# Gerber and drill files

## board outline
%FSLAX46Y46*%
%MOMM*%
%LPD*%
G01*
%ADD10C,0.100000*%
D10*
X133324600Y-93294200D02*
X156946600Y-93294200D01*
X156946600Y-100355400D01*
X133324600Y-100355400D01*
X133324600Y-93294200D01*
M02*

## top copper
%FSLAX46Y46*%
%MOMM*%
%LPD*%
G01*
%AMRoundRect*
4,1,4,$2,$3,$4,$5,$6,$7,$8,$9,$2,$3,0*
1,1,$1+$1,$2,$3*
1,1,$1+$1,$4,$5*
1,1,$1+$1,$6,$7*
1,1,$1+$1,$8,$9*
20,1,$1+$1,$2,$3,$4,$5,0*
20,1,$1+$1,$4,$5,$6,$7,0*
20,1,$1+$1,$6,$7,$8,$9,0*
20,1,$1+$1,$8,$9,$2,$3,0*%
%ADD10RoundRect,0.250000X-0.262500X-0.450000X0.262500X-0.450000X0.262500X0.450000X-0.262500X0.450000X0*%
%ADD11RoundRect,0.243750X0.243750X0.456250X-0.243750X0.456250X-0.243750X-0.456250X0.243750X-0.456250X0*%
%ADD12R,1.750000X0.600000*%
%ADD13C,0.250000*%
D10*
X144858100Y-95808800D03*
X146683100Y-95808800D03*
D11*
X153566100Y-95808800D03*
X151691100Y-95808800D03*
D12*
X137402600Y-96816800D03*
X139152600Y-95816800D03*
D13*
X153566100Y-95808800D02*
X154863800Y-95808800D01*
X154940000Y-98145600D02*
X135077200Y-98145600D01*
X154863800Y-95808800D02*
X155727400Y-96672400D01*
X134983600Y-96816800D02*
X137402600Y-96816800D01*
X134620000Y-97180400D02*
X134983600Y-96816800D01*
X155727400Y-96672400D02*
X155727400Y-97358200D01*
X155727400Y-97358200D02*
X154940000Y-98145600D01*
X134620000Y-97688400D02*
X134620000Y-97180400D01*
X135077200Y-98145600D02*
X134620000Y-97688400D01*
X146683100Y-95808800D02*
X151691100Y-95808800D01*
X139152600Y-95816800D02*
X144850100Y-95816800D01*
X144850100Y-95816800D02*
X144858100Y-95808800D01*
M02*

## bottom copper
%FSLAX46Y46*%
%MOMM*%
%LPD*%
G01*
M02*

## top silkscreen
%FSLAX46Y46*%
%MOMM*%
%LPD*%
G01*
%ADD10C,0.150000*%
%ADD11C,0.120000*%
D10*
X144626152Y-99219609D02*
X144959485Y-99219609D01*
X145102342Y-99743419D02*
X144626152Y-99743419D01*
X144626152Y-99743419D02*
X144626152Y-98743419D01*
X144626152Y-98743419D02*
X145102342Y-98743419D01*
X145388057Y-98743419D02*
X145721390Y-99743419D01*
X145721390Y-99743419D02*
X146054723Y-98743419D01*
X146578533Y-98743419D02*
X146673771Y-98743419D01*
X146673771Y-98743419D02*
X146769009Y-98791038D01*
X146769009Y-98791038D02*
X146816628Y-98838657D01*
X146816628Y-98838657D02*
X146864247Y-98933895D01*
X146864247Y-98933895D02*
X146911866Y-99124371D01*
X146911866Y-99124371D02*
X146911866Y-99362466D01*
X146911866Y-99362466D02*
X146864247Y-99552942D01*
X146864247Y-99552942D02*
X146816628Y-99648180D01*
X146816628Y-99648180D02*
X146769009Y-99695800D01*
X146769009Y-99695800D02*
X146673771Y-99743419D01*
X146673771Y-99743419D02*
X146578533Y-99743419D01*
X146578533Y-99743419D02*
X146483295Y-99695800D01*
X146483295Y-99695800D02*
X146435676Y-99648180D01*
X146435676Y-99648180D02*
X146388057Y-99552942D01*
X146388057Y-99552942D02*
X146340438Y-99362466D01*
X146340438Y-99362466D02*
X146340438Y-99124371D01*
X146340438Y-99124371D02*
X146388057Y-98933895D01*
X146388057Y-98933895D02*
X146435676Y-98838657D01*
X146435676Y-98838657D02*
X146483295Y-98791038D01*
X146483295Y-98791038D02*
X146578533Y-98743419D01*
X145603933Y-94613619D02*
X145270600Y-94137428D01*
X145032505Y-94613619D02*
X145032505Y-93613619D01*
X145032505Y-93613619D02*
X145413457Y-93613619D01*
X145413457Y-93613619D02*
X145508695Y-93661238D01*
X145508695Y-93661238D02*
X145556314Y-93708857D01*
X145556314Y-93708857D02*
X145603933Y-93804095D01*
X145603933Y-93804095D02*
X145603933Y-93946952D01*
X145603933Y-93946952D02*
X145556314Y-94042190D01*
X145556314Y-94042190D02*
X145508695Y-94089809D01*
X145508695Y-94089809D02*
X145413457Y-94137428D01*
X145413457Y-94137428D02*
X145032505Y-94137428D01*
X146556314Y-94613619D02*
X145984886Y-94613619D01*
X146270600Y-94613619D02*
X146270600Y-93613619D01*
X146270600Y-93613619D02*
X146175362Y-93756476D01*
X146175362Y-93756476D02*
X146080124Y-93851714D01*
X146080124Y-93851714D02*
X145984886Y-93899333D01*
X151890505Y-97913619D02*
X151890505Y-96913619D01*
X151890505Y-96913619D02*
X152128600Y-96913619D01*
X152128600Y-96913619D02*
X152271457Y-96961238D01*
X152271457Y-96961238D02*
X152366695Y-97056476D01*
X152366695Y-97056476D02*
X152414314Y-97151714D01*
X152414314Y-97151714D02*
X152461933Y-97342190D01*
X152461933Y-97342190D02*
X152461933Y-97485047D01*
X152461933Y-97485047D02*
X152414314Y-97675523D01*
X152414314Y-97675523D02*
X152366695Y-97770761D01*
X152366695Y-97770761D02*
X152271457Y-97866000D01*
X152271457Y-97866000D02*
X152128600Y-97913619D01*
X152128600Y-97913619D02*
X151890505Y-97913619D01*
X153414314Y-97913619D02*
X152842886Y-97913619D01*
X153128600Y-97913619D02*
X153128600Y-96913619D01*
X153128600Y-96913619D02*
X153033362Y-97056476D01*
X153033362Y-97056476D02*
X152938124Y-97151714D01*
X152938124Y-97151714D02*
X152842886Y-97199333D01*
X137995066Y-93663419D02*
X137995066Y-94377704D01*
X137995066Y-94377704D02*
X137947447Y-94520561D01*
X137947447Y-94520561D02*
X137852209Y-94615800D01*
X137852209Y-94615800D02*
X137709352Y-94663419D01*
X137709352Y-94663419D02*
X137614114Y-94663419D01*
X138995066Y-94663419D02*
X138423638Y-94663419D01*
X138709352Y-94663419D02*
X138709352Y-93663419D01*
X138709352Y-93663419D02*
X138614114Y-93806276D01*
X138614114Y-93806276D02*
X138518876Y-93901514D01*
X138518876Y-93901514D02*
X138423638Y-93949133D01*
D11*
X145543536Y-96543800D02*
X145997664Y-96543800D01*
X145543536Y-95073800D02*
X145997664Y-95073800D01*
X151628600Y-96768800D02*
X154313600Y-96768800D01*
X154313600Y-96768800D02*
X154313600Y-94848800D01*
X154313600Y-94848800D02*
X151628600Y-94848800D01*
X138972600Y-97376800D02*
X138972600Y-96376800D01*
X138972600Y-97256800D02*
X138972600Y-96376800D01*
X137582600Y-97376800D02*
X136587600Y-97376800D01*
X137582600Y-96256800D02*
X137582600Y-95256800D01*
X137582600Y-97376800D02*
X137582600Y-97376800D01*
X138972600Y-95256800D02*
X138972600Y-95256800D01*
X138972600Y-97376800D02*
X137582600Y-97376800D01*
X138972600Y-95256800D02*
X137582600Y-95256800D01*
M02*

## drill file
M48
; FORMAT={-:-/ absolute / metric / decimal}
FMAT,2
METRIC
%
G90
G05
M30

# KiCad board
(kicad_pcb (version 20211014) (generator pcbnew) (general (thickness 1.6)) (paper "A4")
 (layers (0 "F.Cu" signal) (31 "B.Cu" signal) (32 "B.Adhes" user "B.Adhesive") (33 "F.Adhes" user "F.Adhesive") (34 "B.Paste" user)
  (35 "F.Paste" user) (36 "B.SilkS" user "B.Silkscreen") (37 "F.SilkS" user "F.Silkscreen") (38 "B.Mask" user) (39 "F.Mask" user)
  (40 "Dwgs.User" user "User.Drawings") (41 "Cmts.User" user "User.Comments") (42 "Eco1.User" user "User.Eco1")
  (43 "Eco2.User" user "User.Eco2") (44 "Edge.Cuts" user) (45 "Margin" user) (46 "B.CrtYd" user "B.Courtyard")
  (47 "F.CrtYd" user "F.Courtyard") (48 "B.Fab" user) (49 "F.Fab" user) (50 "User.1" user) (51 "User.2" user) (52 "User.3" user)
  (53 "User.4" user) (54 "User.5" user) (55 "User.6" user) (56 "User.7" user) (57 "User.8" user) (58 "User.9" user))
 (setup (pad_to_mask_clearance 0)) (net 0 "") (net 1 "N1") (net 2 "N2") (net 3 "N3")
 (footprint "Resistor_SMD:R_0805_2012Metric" (layer "F.Cu") (at 145.7706 95.8088)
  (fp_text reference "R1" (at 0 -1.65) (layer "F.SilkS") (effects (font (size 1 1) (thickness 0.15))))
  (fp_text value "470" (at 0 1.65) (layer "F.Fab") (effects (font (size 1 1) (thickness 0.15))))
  (fp_line (start -0.227064 0.735) (end 0.227064 0.735) (layer "F.SilkS") (width 0.12))
  (fp_line (start -0.227064 -0.735) (end 0.227064 -0.735) (layer "F.SilkS") (width 0.12))
  (pad "1" smd roundrect (at -0.9125 0) (size 1.025 1.4) (layers "F.Cu" "F.Paste" "F.Mask") (roundrect_rratio 0.243902) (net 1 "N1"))
  (pad "2" smd roundrect (at 0.9125 0) (size 1.025 1.4) (layers "F.Cu" "F.Paste" "F.Mask") (roundrect_rratio 0.243902) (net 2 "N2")))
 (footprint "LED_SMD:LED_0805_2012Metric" (layer "F.Cu") (at 152.6286 95.8088 180)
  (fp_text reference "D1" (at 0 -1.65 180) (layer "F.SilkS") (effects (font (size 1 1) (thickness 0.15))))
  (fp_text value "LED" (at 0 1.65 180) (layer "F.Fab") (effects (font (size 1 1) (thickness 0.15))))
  (fp_line (start 1 -0.96) (end -1.685 -0.96) (layer "F.SilkS") (width 0.12))
  (fp_line (start -1.685 -0.96) (end -1.685 0.96) (layer "F.SilkS") (width 0.12))
  (fp_line (start -1.685 0.96) (end 1 0.96) (layer "F.SilkS") (width 0.12))
  (pad "1" smd roundrect (at -0.9375 0 180) (size 0.975 1.4) (layers "F.Cu" "F.Paste" "F.Mask") (roundrect_rratio 0.25) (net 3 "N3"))
  (pad "2" smd roundrect (at 0.9375 0 180) (size 0.975 1.4) (layers "F.Cu" "F.Paste" "F.Mask") (roundrect_rratio 0.25) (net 2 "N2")))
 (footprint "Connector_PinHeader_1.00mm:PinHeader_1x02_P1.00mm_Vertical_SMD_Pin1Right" (layer "F.Cu") (at 138.2776 96.3168 180)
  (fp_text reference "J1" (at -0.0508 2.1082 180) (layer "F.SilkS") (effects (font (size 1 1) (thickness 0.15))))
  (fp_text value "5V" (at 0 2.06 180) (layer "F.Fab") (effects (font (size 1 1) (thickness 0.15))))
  (fp_line (start -0.695 -1.06) (end -0.695 -0.06) (layer "F.SilkS") (width 0.12))
  (fp_line (start -0.695 -0.94) (end -0.695 -0.06) (layer "F.SilkS") (width 0.12))
  (fp_line (start 0.695 -1.06) (end 1.69 -1.06) (layer "F.SilkS") (width 0.12))
  (fp_line (start 0.695 0.06) (end 0.695 1.06) (layer "F.SilkS") (width 0.12))
  (fp_line (start 0.695 -1.06) (end 0.695 -1.06) (layer "F.SilkS") (width 0.12))
  (fp_line (start -0.695 1.06) (end -0.695 1.06) (layer "F.SilkS") (width 0.12))
  (fp_line (start -0.695 -1.06) (end 0.695 -1.06) (layer "F.SilkS") (width 0.12))
  (fp_line (start -0.695 1.06) (end 0.695 1.06) (layer "F.SilkS") (width 0.12))
  (pad "1" smd rect (at 0.875 -0.5 180) (size 1.75 0.6) (layers "F.Cu" "F.Paste" "F.Mask") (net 3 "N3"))
  (pad "2" smd rect (at -0.875 0.5 180) (size 1.75 0.6) (layers "F.Cu" "F.Paste" "F.Mask") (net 1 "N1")))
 (gr_rect (start 133.3246 93.2942) (end 156.9466 100.3554) (layer "Edge.Cuts") (width 0.1) (fill none))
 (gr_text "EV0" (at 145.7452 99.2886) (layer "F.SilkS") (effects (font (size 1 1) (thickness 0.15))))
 (segment (start 153.5661 95.8088) (end 154.8638 95.8088) (width 0.25) (layer "F.Cu") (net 3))
 (segment (start 154.94 98.1456) (end 135.0772 98.1456) (width 0.25) (layer "F.Cu") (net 3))
 (segment (start 154.8638 95.8088) (end 155.7274 96.6724) (width 0.25) (layer "F.Cu") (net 3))
 (segment (start 134.9836 96.8168) (end 137.4026 96.8168) (width 0.25) (layer "F.Cu") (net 3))
 (segment (start 134.62 97.1804) (end 134.9836 96.8168) (width 0.25) (layer "F.Cu") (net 3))
 (segment (start 155.7274 96.6724) (end 155.7274 97.3582) (width 0.25) (layer "F.Cu") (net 3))
 (segment (start 155.7274 97.3582) (end 154.94 98.1456) (width 0.25) (layer "F.Cu") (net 3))
 (segment (start 134.62 97.6884) (end 134.62 97.1804) (width 0.25) (layer "F.Cu") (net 3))
 (segment (start 135.0772 98.1456) (end 134.62 97.6884) (width 0.25) (layer "F.Cu") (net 3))
 (segment (start 146.6831 95.8088) (end 151.6911 95.8088) (width 0.25) (layer "F.Cu") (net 2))
 (segment (start 139.1526 95.8168) (end 144.8501 95.8168) (width 0.25) (layer "F.Cu") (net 1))
 (segment (start 144.8501 95.8168) (end 144.8581 95.8088) (width 0.25) (layer "F.Cu") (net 1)))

